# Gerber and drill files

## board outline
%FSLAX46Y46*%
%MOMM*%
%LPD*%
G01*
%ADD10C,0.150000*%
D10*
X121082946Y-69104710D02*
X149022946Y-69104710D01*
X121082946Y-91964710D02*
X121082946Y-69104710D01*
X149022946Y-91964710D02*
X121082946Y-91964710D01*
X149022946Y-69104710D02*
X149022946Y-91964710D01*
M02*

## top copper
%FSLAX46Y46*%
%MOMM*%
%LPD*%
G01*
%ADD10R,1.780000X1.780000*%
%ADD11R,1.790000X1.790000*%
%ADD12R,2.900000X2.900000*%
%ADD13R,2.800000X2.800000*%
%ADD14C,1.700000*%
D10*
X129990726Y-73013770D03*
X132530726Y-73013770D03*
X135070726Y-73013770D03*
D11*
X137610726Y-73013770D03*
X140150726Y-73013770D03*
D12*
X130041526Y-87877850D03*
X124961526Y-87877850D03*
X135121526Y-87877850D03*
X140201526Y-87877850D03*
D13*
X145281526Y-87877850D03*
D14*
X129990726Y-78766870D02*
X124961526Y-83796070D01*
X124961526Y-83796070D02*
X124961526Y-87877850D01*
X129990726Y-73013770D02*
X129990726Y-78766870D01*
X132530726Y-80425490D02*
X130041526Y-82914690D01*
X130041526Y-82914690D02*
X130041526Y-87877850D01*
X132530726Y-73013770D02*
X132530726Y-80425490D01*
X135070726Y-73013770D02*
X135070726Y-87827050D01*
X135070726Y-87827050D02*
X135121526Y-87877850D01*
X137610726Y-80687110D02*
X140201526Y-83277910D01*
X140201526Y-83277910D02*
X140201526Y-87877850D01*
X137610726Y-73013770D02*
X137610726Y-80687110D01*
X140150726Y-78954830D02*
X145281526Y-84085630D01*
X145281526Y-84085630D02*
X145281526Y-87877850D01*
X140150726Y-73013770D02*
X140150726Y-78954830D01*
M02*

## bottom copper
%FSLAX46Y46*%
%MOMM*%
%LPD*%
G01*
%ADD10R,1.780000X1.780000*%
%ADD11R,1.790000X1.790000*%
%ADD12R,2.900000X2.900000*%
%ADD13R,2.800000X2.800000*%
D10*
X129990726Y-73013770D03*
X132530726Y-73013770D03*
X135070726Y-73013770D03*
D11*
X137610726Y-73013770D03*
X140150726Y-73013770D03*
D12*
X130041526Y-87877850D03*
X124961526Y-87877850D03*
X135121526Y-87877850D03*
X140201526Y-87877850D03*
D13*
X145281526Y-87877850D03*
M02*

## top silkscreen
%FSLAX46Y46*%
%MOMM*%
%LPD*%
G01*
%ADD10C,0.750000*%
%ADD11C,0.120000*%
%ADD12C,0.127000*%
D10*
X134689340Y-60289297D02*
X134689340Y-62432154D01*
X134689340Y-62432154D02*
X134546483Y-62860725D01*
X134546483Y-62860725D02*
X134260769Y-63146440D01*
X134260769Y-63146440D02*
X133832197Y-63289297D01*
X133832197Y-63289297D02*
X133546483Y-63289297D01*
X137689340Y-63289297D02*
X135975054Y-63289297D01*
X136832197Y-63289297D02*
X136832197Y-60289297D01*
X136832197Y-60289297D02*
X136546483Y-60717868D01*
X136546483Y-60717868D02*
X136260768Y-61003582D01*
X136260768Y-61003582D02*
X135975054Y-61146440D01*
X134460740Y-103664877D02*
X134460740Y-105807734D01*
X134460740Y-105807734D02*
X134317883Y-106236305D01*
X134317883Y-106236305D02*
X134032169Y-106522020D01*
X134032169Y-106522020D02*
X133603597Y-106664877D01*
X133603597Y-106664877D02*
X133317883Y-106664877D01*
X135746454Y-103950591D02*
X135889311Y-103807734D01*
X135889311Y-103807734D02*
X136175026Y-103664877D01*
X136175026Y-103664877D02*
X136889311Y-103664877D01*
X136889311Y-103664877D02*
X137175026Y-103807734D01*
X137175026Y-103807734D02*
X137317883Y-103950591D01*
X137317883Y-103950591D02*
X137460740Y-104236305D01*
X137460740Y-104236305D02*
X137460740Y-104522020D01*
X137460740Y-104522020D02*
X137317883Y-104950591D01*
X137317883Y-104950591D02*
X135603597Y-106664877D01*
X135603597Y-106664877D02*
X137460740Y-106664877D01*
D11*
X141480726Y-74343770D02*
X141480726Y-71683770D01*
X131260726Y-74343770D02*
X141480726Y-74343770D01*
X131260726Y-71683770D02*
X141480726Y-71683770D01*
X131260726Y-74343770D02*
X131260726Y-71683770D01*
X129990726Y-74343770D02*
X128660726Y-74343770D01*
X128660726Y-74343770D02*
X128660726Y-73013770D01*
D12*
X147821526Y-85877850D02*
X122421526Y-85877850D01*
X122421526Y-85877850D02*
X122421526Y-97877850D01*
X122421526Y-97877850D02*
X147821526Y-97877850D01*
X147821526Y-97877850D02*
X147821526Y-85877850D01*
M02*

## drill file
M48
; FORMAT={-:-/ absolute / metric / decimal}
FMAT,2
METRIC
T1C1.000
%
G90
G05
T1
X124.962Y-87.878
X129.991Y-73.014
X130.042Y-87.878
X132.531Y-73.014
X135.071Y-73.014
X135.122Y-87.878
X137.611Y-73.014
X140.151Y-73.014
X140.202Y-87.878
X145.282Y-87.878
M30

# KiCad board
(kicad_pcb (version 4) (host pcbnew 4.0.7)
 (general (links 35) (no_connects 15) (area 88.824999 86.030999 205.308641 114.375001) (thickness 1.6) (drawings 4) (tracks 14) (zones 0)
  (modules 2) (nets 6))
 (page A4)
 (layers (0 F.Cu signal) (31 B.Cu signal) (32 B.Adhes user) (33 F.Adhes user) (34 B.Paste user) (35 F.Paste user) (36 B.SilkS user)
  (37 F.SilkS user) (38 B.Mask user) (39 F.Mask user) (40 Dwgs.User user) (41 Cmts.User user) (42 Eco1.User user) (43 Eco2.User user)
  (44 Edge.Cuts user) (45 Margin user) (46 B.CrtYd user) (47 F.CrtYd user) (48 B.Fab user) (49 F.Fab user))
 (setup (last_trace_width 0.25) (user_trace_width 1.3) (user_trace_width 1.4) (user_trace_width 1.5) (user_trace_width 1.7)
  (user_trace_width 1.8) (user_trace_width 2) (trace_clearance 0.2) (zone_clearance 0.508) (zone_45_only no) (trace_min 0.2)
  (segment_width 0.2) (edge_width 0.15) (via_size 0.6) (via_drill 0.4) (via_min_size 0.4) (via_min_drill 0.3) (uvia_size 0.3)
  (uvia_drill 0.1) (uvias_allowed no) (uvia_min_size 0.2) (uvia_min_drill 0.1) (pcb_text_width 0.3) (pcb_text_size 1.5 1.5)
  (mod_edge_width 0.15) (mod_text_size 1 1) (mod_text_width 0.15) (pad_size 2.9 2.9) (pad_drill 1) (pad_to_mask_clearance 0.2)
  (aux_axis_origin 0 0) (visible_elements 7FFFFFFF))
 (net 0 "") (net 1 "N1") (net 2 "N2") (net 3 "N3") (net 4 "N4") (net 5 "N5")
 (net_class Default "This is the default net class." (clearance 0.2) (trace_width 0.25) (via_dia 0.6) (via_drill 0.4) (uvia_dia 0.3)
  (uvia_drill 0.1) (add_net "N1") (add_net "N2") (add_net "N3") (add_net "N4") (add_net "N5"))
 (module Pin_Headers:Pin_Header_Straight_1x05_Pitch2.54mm (layer F.Cu) (at 129.990726 73.01377 90)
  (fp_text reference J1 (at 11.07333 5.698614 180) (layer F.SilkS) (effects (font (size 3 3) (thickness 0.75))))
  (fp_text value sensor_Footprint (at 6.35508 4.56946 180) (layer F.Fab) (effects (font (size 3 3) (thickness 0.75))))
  (fp_line (start -1.33 11.49) (end 1.33 11.49) (layer F.SilkS) (width 0.12))
  (fp_line (start -1.33 1.27) (end -1.33 11.49) (layer F.SilkS) (width 0.12))
  (fp_line (start 1.33 1.27) (end 1.33 11.49) (layer F.SilkS) (width 0.12))
  (fp_line (start -1.33 1.27) (end 1.33 1.27) (layer F.SilkS) (width 0.12))
  (fp_line (start -1.33 0) (end -1.33 -1.33) (layer F.SilkS) (width 0.12))
  (fp_line (start -1.33 -1.33) (end 0 -1.33) (layer F.SilkS) (width 0.12))
  (pad 1 thru_hole rect (at 0 0 90) (size 1.78 1.78) (drill 1) (layers *.Cu *.Mask) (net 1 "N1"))
  (pad 2 thru_hole rect (at 0 2.54 90) (size 1.78 1.78) (drill 1) (layers *.Cu *.Mask) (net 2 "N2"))
  (pad 3 thru_hole rect (at 0 5.08 90) (size 1.78 1.78) (drill 1) (layers *.Cu *.Mask) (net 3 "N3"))
  (pad 4 thru_hole rect (at 0 7.62 90) (size 1.79 1.79) (drill 1) (layers *.Cu *.Mask) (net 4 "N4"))
  (pad 5 thru_hole rect (at 0 10.16 90) (size 1.79 1.79) (drill 1) (layers *.Cu *.Mask) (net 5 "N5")))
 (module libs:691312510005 (layer F.Cu) (at 135.121526 87.87785)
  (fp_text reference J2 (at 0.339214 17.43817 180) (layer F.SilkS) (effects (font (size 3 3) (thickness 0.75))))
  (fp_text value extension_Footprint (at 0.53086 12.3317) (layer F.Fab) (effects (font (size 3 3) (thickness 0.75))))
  (fp_line (start 12.7 -2) (end -12.7 -2) (layer F.SilkS) (width 0.127))
  (fp_line (start -12.7 -2) (end -12.7 10) (layer F.SilkS) (width 0.127))
  (fp_line (start -12.7 10) (end 12.7 10) (layer F.SilkS) (width 0.127))
  (fp_line (start 12.7 10) (end 12.7 -2) (layer F.SilkS) (width 0.127))
  (pad 2 thru_hole rect (at -5.08 0) (size 2.9 2.9) (drill 1) (layers *.Cu *.Mask) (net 2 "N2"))
  (pad 1 thru_hole rect (at -10.16 0) (size 2.9 2.9) (drill 1) (layers *.Cu *.Mask) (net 1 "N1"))
  (pad 3 thru_hole rect (at 0 0) (size 2.9 2.9) (drill 1) (layers *.Cu *.Mask) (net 3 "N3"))
  (pad 4 thru_hole rect (at 5.08 0) (size 2.9 2.9) (drill 1) (layers *.Cu *.Mask) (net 4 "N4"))
  (pad 5 thru_hole rect (at 10.16 0) (size 2.8 2.8) (drill 1) (layers *.Cu *.Mask) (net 5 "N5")))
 (gr_line (start 121.082946 69.10471) (end 149.022946 69.10471) (layer Edge.Cuts) (width 0.15))
 (gr_line (start 121.082946 91.96471) (end 121.082946 69.10471) (layer Edge.Cuts) (width 0.15))
 (gr_line (start 149.022946 91.96471) (end 121.082946 91.96471) (layer Edge.Cuts) (width 0.15))
 (gr_line (start 149.022946 69.10471) (end 149.022946 91.96471) (layer Edge.Cuts) (width 0.15))
 (segment (start 129.990726 78.76687) (end 124.961526 83.79607) (width 1.7) (layer F.Cu) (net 1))
 (segment (start 124.961526 83.79607) (end 124.961526 87.87785) (width 1.7) (layer F.Cu) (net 1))
 (segment (start 129.990726 73.01377) (end 129.990726 78.76687) (width 1.7) (layer F.Cu) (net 1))
 (segment (start 132.530726 80.42549) (end 130.041526 82.91469) (width 1.7) (layer F.Cu) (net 2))
 (segment (start 130.041526 82.91469) (end 130.041526 87.87785) (width 1.7) (layer F.Cu) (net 2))
 (segment (start 132.530726 73.01377) (end 132.530726 80.42549) (width 1.7) (layer F.Cu) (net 2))
 (segment (start 135.070726 73.01377) (end 135.070726 87.82705) (width 1.7) (layer F.Cu) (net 3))
 (segment (start 135.070726 87.82705) (end 135.121526 87.87785) (width 1.7) (layer F.Cu) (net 3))
 (segment (start 137.610726 80.68711) (end 140.201526 83.27791) (width 1.7) (layer F.Cu) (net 4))
 (segment (start 140.201526 83.27791) (end 140.201526 87.87785) (width 1.7) (layer F.Cu) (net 4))
 (segment (start 137.610726 73.01377) (end 137.610726 80.68711) (width 1.7) (layer F.Cu) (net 4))
 (segment (start 140.150726 78.95483) (end 145.281526 84.08563) (width 1.7) (layer F.Cu) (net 5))
 (segment (start 145.281526 84.08563) (end 145.281526 87.87785) (width 1.7) (layer F.Cu) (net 5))
 (segment (start 140.150726 73.01377) (end 140.150726 78.95483) (width 1.7) (layer F.Cu) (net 5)))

